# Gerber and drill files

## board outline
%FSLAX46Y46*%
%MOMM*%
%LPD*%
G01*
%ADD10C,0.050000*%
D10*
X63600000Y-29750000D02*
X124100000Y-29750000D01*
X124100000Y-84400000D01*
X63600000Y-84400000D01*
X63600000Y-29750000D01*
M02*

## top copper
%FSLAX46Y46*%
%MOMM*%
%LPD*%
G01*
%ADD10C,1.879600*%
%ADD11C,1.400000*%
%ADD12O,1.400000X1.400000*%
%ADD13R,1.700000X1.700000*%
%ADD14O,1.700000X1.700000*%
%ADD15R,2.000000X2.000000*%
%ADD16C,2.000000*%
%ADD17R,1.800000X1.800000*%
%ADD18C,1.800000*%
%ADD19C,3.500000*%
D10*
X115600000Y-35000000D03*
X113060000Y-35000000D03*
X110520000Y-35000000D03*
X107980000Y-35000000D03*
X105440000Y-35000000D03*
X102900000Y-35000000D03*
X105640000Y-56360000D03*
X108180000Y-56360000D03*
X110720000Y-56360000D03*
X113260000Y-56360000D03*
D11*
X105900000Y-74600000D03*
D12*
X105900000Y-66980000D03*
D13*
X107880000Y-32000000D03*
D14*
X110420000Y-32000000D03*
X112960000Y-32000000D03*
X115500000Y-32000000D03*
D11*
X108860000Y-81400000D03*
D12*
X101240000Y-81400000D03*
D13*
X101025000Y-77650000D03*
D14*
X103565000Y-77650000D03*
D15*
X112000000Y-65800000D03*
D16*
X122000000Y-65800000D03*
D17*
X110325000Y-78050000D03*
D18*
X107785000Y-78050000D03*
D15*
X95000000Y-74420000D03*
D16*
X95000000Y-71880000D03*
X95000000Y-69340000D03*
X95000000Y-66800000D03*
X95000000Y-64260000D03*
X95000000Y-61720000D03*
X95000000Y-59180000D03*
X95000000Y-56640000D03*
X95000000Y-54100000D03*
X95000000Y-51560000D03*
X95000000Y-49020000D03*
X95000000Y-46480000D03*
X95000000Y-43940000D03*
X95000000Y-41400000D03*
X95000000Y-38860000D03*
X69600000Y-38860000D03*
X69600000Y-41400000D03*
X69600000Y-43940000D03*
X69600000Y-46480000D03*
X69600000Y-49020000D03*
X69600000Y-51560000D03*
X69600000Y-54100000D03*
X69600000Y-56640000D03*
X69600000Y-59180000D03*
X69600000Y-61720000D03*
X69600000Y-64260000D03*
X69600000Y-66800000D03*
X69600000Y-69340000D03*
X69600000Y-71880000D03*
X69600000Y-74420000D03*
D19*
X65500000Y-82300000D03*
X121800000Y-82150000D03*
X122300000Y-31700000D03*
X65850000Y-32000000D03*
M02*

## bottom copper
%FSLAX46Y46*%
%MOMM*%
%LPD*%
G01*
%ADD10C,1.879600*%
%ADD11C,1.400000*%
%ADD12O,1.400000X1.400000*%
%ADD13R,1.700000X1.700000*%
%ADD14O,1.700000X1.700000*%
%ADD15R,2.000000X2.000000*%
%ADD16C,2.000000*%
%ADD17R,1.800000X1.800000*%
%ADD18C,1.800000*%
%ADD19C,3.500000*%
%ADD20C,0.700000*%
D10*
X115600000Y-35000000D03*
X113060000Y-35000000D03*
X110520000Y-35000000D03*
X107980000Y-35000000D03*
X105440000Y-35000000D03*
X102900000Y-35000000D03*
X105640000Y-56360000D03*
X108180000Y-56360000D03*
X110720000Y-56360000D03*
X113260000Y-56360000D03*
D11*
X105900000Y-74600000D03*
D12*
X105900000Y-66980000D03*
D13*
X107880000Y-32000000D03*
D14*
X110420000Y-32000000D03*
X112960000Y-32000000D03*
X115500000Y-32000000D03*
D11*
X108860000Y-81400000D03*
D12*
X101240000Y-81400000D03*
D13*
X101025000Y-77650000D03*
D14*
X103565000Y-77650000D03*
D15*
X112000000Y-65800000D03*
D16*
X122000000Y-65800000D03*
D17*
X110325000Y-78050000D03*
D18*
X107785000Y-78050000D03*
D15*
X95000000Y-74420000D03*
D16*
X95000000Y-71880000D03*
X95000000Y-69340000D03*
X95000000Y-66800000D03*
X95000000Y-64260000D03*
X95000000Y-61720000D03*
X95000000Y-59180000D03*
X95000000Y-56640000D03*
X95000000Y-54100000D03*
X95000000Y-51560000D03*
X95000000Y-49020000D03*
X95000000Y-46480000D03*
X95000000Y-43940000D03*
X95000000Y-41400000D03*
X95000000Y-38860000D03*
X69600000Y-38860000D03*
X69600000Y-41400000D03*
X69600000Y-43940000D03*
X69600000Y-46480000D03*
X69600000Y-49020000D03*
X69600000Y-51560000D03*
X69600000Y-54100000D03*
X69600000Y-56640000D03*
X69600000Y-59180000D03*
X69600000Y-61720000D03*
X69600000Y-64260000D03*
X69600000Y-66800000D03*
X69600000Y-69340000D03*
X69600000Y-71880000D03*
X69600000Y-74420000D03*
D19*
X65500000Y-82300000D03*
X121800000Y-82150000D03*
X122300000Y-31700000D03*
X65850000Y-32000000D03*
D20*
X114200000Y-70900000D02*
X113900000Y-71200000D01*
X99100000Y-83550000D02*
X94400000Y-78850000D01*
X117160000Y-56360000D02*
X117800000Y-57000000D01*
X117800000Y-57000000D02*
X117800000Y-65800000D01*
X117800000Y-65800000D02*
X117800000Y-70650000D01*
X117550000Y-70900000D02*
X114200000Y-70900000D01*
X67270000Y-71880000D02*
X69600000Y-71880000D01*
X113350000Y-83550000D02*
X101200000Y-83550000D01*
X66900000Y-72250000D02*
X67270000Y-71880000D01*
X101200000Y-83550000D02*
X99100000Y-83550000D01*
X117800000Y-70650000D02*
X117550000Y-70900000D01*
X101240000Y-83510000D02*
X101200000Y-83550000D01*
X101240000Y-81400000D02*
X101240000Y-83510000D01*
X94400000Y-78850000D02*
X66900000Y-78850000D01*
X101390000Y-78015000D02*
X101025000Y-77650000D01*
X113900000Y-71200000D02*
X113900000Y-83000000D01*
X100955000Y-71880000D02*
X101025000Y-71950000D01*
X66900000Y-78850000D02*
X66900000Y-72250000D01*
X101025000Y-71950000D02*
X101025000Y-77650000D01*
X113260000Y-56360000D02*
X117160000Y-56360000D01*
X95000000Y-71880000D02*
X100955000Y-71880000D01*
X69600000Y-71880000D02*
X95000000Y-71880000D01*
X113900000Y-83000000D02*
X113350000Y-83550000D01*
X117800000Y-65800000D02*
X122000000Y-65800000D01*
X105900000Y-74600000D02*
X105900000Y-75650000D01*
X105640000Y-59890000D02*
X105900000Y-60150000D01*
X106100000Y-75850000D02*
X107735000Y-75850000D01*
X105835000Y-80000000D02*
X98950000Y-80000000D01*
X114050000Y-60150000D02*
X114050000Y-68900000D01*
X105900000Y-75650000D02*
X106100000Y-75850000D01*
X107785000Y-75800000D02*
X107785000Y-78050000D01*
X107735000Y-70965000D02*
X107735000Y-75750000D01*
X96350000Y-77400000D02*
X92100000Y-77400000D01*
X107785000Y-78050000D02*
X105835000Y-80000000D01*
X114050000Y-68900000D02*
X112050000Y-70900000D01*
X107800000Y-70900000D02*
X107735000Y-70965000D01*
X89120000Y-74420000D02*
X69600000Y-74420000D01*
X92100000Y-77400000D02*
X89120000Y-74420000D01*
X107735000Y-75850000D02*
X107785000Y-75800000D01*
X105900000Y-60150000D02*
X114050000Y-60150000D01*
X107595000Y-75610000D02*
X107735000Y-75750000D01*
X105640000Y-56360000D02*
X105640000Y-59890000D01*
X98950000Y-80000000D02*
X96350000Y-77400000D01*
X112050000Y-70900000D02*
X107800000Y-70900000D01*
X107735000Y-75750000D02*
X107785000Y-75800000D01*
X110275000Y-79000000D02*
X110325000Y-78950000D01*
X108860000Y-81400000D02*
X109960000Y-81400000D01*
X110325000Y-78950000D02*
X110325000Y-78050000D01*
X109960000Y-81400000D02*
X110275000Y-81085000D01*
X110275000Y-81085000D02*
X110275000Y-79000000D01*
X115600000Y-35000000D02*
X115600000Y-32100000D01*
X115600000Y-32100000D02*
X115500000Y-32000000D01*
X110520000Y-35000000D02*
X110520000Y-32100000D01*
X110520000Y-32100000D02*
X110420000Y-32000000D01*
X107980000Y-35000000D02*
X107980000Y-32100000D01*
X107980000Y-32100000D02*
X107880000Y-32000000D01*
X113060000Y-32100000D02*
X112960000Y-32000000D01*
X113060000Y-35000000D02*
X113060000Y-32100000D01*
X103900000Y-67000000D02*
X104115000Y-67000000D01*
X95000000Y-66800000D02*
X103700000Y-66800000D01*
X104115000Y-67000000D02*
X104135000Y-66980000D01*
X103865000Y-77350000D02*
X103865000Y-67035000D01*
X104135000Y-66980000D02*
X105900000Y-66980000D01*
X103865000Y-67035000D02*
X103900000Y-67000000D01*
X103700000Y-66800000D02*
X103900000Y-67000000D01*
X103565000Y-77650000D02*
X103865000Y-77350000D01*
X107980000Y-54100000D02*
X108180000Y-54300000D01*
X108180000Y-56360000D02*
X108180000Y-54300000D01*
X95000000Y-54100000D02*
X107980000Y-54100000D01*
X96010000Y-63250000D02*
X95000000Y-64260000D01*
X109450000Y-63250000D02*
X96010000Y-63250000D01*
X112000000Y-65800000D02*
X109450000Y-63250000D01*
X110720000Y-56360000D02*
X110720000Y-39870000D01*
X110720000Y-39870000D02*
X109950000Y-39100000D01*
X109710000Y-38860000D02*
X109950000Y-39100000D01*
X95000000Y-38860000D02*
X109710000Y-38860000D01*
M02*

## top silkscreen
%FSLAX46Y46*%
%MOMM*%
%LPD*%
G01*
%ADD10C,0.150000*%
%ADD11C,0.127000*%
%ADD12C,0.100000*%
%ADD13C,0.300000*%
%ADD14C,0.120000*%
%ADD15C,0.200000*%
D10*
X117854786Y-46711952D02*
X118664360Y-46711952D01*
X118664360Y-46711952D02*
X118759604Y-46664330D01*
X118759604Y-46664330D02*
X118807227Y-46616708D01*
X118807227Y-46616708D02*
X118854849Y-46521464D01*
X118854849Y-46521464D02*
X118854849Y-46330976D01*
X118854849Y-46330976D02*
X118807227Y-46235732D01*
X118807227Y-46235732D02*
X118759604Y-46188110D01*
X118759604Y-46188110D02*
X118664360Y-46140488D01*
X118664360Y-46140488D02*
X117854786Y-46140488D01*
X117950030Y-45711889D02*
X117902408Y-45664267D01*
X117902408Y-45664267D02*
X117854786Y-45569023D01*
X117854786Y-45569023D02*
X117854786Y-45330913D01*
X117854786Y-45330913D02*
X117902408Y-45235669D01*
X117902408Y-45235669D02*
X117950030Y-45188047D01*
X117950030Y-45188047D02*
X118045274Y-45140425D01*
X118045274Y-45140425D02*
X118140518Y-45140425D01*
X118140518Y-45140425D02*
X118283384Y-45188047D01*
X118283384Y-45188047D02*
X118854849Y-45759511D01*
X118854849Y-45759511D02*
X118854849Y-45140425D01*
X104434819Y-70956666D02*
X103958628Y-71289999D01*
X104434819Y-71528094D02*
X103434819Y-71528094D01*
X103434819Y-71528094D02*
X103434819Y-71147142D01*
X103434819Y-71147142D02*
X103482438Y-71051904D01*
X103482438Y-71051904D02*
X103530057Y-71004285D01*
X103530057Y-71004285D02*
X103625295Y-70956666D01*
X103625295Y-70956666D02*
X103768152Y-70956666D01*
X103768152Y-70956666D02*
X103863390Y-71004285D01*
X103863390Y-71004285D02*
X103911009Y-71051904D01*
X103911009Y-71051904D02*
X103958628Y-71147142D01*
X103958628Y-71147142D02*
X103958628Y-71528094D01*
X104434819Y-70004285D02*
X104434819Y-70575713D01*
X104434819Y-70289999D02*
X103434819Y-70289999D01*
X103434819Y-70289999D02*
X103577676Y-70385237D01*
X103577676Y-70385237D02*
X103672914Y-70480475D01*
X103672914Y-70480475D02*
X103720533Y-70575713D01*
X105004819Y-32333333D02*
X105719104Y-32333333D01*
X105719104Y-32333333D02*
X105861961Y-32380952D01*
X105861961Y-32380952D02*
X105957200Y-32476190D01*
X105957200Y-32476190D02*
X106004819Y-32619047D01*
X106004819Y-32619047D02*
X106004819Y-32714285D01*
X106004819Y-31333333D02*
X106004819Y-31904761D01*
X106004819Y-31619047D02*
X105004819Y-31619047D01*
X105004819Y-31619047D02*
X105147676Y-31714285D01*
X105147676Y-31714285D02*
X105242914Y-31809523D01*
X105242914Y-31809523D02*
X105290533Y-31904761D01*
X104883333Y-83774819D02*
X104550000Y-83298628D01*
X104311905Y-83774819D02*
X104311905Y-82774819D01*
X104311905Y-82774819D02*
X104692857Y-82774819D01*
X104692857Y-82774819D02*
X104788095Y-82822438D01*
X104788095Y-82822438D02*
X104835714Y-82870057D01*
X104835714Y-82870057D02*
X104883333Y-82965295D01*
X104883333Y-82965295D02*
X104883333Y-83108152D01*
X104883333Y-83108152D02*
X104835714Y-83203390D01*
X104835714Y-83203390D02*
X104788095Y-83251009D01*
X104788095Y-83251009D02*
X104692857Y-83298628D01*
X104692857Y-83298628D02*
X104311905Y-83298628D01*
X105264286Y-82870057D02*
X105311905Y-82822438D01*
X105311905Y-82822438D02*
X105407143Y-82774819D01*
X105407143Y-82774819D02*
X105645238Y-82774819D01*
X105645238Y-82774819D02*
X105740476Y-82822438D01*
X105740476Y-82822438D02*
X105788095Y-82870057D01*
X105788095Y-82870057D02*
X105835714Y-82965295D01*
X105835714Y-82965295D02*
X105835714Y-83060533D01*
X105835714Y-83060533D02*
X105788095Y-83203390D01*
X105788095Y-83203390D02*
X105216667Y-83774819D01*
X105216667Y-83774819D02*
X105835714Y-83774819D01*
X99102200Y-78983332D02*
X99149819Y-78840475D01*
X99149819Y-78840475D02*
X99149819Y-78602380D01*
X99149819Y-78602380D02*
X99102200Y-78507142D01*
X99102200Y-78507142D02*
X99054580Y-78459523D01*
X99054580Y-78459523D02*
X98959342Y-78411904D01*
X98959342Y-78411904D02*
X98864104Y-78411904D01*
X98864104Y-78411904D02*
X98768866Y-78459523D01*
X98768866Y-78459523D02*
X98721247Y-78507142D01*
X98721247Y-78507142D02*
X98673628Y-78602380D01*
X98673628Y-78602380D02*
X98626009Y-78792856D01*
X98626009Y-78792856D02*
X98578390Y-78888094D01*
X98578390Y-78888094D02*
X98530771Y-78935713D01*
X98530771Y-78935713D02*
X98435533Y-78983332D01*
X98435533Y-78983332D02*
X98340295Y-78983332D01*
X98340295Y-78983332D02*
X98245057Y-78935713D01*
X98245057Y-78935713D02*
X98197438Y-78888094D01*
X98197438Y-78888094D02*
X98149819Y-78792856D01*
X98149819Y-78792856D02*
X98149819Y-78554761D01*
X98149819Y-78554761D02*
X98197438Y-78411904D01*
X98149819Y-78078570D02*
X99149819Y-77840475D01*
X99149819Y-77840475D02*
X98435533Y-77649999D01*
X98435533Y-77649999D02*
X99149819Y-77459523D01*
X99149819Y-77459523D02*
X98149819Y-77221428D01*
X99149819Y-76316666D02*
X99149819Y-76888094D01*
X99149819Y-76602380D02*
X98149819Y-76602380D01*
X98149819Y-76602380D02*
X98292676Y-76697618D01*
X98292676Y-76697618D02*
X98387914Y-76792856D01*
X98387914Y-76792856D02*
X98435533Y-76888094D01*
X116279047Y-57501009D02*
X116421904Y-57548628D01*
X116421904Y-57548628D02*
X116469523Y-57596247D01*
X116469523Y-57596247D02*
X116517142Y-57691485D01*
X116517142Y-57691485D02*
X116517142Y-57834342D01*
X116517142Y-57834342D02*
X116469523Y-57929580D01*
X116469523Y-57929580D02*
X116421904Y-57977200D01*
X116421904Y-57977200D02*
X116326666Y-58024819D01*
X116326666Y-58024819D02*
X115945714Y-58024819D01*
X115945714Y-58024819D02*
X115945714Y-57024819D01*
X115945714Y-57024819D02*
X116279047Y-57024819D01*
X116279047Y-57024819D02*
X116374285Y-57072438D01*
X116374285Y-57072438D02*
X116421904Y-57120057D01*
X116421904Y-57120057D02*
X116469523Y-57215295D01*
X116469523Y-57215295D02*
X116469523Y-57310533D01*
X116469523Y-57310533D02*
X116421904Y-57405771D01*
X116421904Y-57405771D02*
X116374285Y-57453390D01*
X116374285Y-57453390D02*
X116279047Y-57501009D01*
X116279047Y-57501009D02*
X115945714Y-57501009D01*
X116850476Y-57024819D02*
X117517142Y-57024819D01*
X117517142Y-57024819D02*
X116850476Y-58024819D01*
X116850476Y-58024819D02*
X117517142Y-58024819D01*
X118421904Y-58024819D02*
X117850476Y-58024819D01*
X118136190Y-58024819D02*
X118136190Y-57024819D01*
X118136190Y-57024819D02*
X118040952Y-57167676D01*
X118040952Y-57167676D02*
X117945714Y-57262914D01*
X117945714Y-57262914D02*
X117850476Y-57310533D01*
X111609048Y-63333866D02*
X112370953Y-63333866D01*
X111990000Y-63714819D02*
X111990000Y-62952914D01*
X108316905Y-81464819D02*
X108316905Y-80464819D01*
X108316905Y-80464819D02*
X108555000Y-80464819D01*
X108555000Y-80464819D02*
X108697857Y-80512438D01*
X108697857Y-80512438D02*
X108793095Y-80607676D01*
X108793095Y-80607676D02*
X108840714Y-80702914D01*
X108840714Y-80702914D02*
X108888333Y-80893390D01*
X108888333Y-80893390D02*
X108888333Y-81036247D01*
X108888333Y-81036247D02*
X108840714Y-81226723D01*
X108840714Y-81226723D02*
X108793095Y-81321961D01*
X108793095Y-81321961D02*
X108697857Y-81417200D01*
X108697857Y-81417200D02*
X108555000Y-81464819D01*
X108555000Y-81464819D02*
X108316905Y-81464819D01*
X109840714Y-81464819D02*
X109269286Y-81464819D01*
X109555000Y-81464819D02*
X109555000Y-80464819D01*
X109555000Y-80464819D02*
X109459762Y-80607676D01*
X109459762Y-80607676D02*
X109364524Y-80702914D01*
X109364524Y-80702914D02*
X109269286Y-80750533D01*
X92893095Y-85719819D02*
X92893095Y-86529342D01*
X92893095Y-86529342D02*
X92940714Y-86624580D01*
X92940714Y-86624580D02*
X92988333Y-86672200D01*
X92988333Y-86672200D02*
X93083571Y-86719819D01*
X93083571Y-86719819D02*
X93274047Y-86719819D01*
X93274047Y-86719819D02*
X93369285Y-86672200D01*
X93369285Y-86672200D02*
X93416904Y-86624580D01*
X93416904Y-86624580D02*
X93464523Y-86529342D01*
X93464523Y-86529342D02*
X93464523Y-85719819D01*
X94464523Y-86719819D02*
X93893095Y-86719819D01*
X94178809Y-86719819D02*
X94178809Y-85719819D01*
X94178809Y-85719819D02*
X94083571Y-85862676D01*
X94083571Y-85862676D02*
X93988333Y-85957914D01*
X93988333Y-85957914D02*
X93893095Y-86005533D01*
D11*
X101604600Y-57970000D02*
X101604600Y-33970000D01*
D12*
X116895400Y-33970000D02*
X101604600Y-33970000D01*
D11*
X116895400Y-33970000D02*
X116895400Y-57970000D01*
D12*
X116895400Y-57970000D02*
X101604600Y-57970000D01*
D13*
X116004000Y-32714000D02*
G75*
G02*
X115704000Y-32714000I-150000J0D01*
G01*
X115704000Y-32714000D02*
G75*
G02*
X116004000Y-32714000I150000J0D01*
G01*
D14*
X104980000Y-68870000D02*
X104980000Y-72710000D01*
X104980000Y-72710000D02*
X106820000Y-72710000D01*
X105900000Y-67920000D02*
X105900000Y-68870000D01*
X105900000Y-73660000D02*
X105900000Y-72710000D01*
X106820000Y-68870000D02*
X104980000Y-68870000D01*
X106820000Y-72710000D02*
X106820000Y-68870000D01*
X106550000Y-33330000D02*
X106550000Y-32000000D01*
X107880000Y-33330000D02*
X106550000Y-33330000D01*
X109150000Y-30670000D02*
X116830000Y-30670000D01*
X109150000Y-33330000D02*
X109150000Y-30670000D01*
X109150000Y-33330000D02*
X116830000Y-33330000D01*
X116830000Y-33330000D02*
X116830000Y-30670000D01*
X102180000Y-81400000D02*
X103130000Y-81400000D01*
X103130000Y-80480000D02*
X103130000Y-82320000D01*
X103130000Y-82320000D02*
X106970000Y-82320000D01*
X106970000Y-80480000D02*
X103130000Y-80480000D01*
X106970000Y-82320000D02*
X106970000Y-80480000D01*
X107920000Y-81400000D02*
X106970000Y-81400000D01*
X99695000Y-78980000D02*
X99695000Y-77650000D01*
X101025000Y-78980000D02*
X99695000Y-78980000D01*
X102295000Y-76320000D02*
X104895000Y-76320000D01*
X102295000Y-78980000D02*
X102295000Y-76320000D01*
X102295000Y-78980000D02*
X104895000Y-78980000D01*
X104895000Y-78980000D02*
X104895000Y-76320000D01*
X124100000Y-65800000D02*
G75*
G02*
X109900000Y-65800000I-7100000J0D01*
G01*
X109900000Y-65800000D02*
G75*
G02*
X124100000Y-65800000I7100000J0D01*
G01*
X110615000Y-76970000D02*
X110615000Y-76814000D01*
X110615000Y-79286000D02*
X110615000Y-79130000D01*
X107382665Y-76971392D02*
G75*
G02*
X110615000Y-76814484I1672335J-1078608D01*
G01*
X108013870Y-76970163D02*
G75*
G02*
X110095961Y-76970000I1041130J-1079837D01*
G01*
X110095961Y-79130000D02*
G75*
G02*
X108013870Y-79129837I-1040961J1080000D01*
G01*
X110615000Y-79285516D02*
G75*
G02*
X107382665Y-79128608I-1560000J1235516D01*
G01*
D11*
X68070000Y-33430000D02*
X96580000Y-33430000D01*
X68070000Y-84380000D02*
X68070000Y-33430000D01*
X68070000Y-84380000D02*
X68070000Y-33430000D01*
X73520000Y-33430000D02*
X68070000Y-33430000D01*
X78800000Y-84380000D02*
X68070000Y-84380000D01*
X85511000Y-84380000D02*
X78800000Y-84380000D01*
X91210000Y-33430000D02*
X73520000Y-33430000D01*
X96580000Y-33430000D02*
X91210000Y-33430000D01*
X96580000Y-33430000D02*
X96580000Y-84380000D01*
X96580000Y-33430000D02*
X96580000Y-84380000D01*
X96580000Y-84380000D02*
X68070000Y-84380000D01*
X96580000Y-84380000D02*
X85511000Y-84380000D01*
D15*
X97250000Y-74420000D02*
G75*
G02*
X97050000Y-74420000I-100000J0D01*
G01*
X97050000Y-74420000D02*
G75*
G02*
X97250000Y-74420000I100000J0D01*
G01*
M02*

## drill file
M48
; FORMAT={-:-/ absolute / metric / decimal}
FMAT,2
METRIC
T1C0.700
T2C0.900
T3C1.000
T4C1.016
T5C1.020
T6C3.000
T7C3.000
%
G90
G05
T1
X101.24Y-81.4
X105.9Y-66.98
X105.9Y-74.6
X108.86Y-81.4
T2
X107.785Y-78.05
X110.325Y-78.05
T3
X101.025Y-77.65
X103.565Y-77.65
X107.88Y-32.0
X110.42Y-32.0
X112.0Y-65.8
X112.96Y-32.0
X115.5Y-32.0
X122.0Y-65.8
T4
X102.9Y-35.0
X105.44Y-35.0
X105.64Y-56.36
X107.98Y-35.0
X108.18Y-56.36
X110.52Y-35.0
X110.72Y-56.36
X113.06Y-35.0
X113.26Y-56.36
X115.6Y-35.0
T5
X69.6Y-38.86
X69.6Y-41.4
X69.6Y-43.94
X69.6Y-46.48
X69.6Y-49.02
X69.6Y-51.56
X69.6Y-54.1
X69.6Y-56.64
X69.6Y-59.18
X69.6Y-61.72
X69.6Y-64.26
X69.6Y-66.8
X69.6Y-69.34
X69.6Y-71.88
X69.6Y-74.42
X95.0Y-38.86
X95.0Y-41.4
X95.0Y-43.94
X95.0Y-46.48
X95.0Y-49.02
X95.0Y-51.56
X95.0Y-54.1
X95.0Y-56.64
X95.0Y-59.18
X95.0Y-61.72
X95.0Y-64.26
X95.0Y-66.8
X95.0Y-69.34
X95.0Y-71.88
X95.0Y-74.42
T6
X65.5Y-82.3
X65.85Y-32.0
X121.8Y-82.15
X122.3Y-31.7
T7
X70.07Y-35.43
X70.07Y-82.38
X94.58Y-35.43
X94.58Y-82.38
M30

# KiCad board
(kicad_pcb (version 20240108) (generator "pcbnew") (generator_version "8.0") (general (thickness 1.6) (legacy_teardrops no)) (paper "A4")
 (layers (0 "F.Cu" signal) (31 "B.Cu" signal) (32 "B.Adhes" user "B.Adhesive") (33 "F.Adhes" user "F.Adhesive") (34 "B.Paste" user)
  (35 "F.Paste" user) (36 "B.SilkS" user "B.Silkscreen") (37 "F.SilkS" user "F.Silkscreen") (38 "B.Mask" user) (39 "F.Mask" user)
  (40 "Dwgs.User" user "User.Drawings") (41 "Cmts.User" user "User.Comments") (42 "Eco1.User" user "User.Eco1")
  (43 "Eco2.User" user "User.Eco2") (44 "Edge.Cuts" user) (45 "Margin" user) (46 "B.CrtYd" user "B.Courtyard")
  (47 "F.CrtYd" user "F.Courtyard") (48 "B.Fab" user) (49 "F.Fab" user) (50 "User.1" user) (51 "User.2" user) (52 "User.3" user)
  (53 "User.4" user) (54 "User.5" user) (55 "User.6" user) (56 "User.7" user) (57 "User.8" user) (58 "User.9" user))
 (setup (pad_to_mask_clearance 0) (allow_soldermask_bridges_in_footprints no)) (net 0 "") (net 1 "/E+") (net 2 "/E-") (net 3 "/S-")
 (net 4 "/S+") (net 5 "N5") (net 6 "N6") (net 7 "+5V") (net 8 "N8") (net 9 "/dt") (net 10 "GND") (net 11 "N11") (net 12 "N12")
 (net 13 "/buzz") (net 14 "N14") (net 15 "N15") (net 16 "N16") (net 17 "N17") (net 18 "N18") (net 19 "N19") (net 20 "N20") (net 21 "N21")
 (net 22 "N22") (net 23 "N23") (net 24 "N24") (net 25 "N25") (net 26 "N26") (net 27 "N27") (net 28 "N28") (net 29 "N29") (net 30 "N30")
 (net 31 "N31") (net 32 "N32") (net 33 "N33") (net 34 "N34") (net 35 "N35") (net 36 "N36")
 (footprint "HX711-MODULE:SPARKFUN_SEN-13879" (layer "F.Cu") (at 110.52 48.97 -90)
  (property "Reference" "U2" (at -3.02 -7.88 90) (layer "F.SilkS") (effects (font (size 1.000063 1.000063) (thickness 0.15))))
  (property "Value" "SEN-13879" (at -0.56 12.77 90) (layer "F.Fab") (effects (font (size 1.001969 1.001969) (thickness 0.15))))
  (fp_line (start 9 8.9154) (end -15 8.9154) (stroke (width 0.127) (type solid)) (layer "F.SilkS"))
  (fp_line (start -15 -6.3754) (end -15 8.9154) (stroke (width 0.1) (type default)) (layer "F.SilkS"))
  (fp_line (start -15 -6.3754) (end 9 -6.3754) (stroke (width 0.127) (type solid)) (layer "F.SilkS"))
  (fp_line (start 9 -6.3754) (end 9 8.9154) (stroke (width 0.1) (type default)) (layer "F.SilkS"))
  (fp_circle (center -16.256 -5.334) (end -16.106 -5.334) (stroke (width 0.3) (type solid)) (fill none) (layer "F.SilkS"))
  (pad "1" thru_hole circle (at -13.97 -5.08 270) (size 1.8796 1.8796) (drill 1.016) (layers "*.Cu" "*.Mask") (remove_unused_layers no)
   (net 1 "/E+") (solder_mask_margin 0.102))
  (pad "2" thru_hole circle (at -13.97 -2.54 270) (size 1.8796 1.8796) (drill 1.016) (layers "*.Cu" "*.Mask") (remove_unused_layers no)
   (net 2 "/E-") (solder_mask_margin 0.102))
  (pad "3" thru_hole circle (at -13.97 0 270) (size 1.8796 1.8796) (drill 1.016) (layers "*.Cu" "*.Mask") (remove_unused_layers no)
   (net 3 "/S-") (solder_mask_margin 0.102))
  (pad "4" thru_hole circle (at -13.97 2.54 270) (size 1.8796 1.8796) (drill 1.016) (layers "*.Cu" "*.Mask") (remove_unused_layers no)
   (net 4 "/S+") (solder_mask_margin 0.102))
  (pad "5" thru_hole circle (at -13.97 5.08 270) (size 1.8796 1.8796) (drill 1.016) (layers "*.Cu" "*.Mask") (remove_unused_layers no)
   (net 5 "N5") (solder_mask_margin 0.102))
  (pad "6" thru_hole circle (at -13.97 7.62 270) (size 1.8796 1.8796) (drill 1.016) (layers "*.Cu" "*.Mask") (remove_unused_layers no)
   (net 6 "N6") (solder_mask_margin 0.102))
  (pad "7" thru_hole circle (at 7.39 4.88 270) (size 1.8796 1.8796) (drill 1.016) (layers "*.Cu" "*.Mask") (remove_unused_layers no)
   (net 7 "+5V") (solder_mask_margin 0.102))
  (pad "8" thru_hole circle (at 7.39 2.34 270) (size 1.8796 1.8796) (drill 1.016) (layers "*.Cu" "*.Mask") (remove_unused_layers no)
   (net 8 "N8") (solder_mask_margin 0.102))
  (pad "9" thru_hole circle (at 7.39 -0.2 270) (size 1.8796 1.8796) (drill 1.016) (layers "*.Cu" "*.Mask") (remove_unused_layers no)
   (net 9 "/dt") (solder_mask_margin 0.102))
  (pad "10" thru_hole circle (at 7.39 -2.74 270) (size 1.8796 1.8796) (drill 1.016) (layers "*.Cu" "*.Mask") (remove_unused_layers no)
   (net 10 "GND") (solder_mask_margin 0.102)))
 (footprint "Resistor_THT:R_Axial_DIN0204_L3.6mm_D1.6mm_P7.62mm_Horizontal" (layer "F.Cu") (at 105.9 74.6 90)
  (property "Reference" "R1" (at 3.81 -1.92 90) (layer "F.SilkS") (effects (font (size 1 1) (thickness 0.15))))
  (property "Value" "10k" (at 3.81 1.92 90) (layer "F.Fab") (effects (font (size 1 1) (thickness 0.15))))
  (fp_line (start 5.73 -0.92) (end 1.89 -0.92) (stroke (width 0.12) (type solid)) (layer "F.SilkS"))
  (fp_line (start 1.89 -0.92) (end 1.89 0.92) (stroke (width 0.12) (type solid)) (layer "F.SilkS"))
  (fp_line (start 6.68 0) (end 5.73 0) (stroke (width 0.12) (type solid)) (layer "F.SilkS"))
  (fp_line (start 0.94 0) (end 1.89 0) (stroke (width 0.12) (type solid)) (layer "F.SilkS"))
  (fp_line (start 5.73 0.92) (end 5.73 -0.92) (stroke (width 0.12) (type solid)) (layer "F.SilkS"))
  (fp_line (start 1.89 0.92) (end 5.73 0.92) (stroke (width 0.12) (type solid)) (layer "F.SilkS"))
  (pad "1" thru_hole circle (at 0 0 90) (size 1.4 1.4) (drill 0.7) (layers "*.Cu" "*.Mask") (remove_unused_layers no) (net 7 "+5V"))
  (pad "2" thru_hole oval (at 7.62 0 90) (size 1.4 1.4) (drill 0.7) (layers "*.Cu" "*.Mask") (remove_unused_layers no) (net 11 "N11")))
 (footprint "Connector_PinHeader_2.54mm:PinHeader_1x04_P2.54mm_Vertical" (layer "F.Cu") (at 107.88 32 90)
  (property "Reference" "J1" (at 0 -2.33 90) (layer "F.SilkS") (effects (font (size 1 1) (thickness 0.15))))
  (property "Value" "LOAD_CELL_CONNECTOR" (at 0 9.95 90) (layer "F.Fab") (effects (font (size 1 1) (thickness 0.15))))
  (fp_line (start -1.33 -1.33) (end 0 -1.33) (stroke (width 0.12) (type solid)) (layer "F.SilkS"))
  (fp_line (start -1.33 0) (end -1.33 -1.33) (stroke (width 0.12) (type solid)) (layer "F.SilkS"))
  (fp_line (start 1.33 1.27) (end 1.33 8.95) (stroke (width 0.12) (type solid)) (layer "F.SilkS"))
  (fp_line (start -1.33 1.27) (end 1.33 1.27) (stroke (width 0.12) (type solid)) (layer "F.SilkS"))
  (fp_line (start -1.33 1.27) (end -1.33 8.95) (stroke (width 0.12) (type solid)) (layer "F.SilkS"))
  (fp_line (start -1.33 8.95) (end 1.33 8.95) (stroke (width 0.12) (type solid)) (layer "F.SilkS"))
  (pad "1" thru_hole rect (at 0 0 90) (size 1.7 1.7) (drill 1) (layers "*.Cu" "*.Mask") (remove_unused_layers no) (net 4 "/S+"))
  (pad "2" thru_hole oval (at 0 2.54 90) (size 1.7 1.7) (drill 1) (layers "*.Cu" "*.Mask") (remove_unused_layers no) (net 3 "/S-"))
  (pad "3" thru_hole oval (at 0 5.08 90) (size 1.7 1.7) (drill 1) (layers "*.Cu" "*.Mask") (remove_unused_layers no) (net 2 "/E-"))
  (pad "4" thru_hole oval (at 0 7.62 90) (size 1.7 1.7) (drill 1) (layers "*.Cu" "*.Mask") (remove_unused_layers no) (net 1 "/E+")))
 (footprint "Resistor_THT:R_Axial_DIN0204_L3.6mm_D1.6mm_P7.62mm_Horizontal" (layer "F.Cu") (at 108.86 81.4 180)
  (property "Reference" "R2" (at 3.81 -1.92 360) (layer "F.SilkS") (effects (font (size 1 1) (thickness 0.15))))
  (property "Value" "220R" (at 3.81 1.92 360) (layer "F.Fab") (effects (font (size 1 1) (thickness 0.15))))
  (fp_line (start 6.68 0) (end 5.73 0) (stroke (width 0.12) (type solid)) (layer "F.SilkS"))
  (fp_line (start 5.73 0.92) (end 5.73 -0.92) (stroke (width 0.12) (type solid)) (layer "F.SilkS"))
  (fp_line (start 5.73 -0.92) (end 1.89 -0.92) (stroke (width 0.12) (type solid)) (layer "F.SilkS"))
  (fp_line (start 1.89 0.92) (end 5.73 0.92) (stroke (width 0.12) (type solid)) (layer "F.SilkS"))
  (fp_line (start 1.89 -0.92) (end 1.89 0.92) (stroke (width 0.12) (type solid)) (layer "F.SilkS"))
  (fp_line (start 0.94 0) (end 1.89 0) (stroke (width 0.12) (type solid)) (layer "F.SilkS"))
  (pad "1" thru_hole circle (at 0 0 180) (size 1.4 1.4) (drill 0.7) (layers "*.Cu" "*.Mask") (remove_unused_layers no) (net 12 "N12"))
  (pad "2" thru_hole oval (at 7.62 0 180) (size 1.4 1.4) (drill 0.7) (layers "*.Cu" "*.Mask") (remove_unused_layers no) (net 10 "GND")))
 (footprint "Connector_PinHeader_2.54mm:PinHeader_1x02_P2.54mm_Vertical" (layer "F.Cu") (at 101.025 77.65 90)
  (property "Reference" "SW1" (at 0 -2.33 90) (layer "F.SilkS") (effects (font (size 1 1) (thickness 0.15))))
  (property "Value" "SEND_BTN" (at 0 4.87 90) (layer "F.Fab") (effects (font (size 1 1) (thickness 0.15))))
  (fp_line (start -1.33 -1.33) (end 0 -1.33) (stroke (width 0.12) (type solid)) (layer "F.SilkS"))
  (fp_line (start -1.33 0) (end -1.33 -1.33) (stroke (width 0.12) (type solid)) (layer "F.SilkS"))
  (fp_line (start 1.33 1.27) (end 1.33 3.87) (stroke (width 0.12) (type solid)) (layer "F.SilkS"))
  (fp_line (start -1.33 1.27) (end 1.33 1.27) (stroke (width 0.12) (type solid)) (layer "F.SilkS"))
  (fp_line (start -1.33 1.27) (end -1.33 3.87) (stroke (width 0.12) (type solid)) (layer "F.SilkS"))
  (fp_line (start -1.33 3.87) (end 1.33 3.87) (stroke (width 0.12) (type solid)) (layer "F.SilkS"))
  (pad "1" thru_hole rect (at 0 0 90) (size 1.7 1.7) (drill 1) (layers "*.Cu" "*.Mask") (remove_unused_layers no) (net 10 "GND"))
  (pad "2" thru_hole oval (at 0 2.54 90) (size 1.7 1.7) (drill 1) (layers "*.Cu" "*.Mask") (remove_unused_layers no) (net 11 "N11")))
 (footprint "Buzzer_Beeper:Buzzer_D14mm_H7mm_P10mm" (layer "F.Cu") (at 112 65.8)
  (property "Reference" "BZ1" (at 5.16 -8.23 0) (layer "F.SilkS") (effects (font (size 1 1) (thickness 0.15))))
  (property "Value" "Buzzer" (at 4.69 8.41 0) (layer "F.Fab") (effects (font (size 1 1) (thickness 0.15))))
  (fp_circle (center 5 0) (end 12.1 0) (stroke (width 0.12) (type solid)) (fill none) (layer "F.SilkS"))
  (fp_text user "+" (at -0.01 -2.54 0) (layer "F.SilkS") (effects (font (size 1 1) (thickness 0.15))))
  (pad "1" thru_hole rect (at 0 0) (size 2 2) (drill 1) (layers "*.Cu" "*.Mask") (remove_unused_layers no) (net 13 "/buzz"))
  (pad "2" thru_hole circle (at 10 0) (size 2 2) (drill 1) (layers "*.Cu" "*.Mask") (remove_unused_layers no) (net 10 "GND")))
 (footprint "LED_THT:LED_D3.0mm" (layer "F.Cu") (at 110.325 78.05 180)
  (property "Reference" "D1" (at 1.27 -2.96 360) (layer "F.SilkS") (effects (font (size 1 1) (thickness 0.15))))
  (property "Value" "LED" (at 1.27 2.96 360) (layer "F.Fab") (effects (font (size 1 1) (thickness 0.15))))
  (fp_line (start -0.29 1.08) (end -0.29 1.236) (stroke (width 0.12) (type solid)) (layer "F.SilkS"))
  (fp_line (start -0.29 -1.236) (end -0.29 -1.08) (stroke (width 0.12) (type solid)) (layer "F.SilkS"))
  (fp_arc (start 2.942335 1.078608) (mid 1.366487 1.987659) (end -0.29 1.235516) (stroke (width 0.12) (type solid)) (layer "F.SilkS"))
  (fp_arc (start 2.31113 1.079837) (mid 1.270117 1.5) (end 0.229039 1.08) (stroke (width 0.12) (type solid)) (layer "F.SilkS"))
  (fp_arc (start 0.229039 -1.08) (mid 1.270117 -1.5) (end 2.31113 -1.079837) (stroke (width 0.12) (type solid)) (layer "F.SilkS"))
  (fp_arc (start -0.29 -1.235516) (mid 1.366487 -1.987659) (end 2.942335 -1.078608) (stroke (width 0.12) (type solid)) (layer "F.SilkS"))
  (pad "1" thru_hole rect (at 0 0 180) (size 1.8 1.8) (drill 0.9) (layers "*.Cu" "*.Mask") (remove_unused_layers no) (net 12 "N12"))
  (pad "2" thru_hole circle (at 2.54 0 180) (size 1.8 1.8) (drill 0.9) (layers "*.Cu" "*.Mask") (remove_unused_layers no) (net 7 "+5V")))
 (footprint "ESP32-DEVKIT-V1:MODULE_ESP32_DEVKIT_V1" (layer "F.Cu") (at 82.3 58.905 180)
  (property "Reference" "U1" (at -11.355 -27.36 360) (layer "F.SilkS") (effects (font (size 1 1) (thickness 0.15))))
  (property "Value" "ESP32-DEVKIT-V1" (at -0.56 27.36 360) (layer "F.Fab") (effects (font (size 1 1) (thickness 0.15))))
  (fp_line (start 14.23 25.475) (end -14.28 25.475) (stroke (width 0.127) (type solid)) (layer "F.SilkS"))
  (fp_line (start 14.23 -25.475) (end 14.23 25.475) (stroke (width 0.127) (type solid)) (layer "F.SilkS"))
  (fp_line (start 14.23 -25.475) (end 14.23 25.475) (stroke (width 0.127) (type solid)) (layer "F.SilkS"))
  (fp_line (start 8.78 25.475) (end 14.23 25.475) (stroke (width 0.127) (type solid)) (layer "F.SilkS"))
  (fp_line (start 3.5 -25.475) (end 14.23 -25.475) (stroke (width 0.127) (type solid)) (layer "F.SilkS"))
  (fp_line (start -3.211 -25.475) (end 3.5 -25.475) (stroke (width 0.127) (type solid)) (layer "F.SilkS"))
  (fp_line (start -8.91 25.475) (end 8.78 25.475) (stroke (width 0.127) (type solid)) (layer "F.SilkS"))
  (fp_line (start -14.28 25.475) (end -8.91 25.475) (stroke (width 0.127) (type solid)) (layer "F.SilkS"))
  (fp_line (start -14.28 25.475) (end -14.28 -25.475) (stroke (width 0.127) (type solid)) (layer "F.SilkS"))
  (fp_line (start -14.28 25.475) (end -14.28 -25.475) (stroke (width 0.127) (type solid)) (layer "F.SilkS"))
  (fp_line (start -14.28 -25.475) (end 14.23 -25.475) (stroke (width 0.127) (type solid)) (layer "F.SilkS"))
  (fp_line (start -14.28 -25.475) (end -3.211 -25.475) (stroke (width 0.127) (type solid)) (layer "F.SilkS"))
  (fp_circle (center -14.85 -15.515) (end -14.75 -15.515) (stroke (width 0.2) (type solid)) (fill none) (layer "F.SilkS"))
  (pad "" np_thru_hole circle (at -12.28 -23.475 180) (size 3 3) (drill 3) (layers "*.Cu" "*.Mask"))
  (pad "" np_thru_hole circle (at -12.28 23.475 180) (size 3 3) (drill 3) (layers "*.Cu" "*.Mask"))
  (pad "" np_thru_hole circle (at 12.23 -23.475 180) (size 3 3) (drill 3) (layers "*.Cu" "*.Mask"))
  (pad "" np_thru_hole circle (at 12.23 23.475 180) (size 3 3) (drill 3) (layers "*.Cu" "*.Mask"))
  (pad "1" thru_hole rect (at -12.7 -15.515 180) (size 2 2) (drill 1.02) (layers "*.Cu" "*.Mask") (remove_unused_layers no) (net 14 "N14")
   (solder_mask_margin 0.102))
  (pad "2" thru_hole circle (at -12.7 -12.975 180) (size 2 2) (drill 1.02) (layers "*.Cu" "*.Mask") (remove_unused_layers no) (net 10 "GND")
   (solder_mask_margin 0.102))
  (pad "3" thru_hole circle (at -12.7 -10.435 180) (size 2 2) (drill 1.02) (layers "*.Cu" "*.Mask") (remove_unused_layers no) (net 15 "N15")
   (solder_mask_margin 0.102))
  (pad "4" thru_hole circle (at -12.7 -7.895 180) (size 2 2) (drill 1.02) (layers "*.Cu" "*.Mask") (remove_unused_layers no) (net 11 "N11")
   (solder_mask_margin 0.102))
  (pad "5" thru_hole circle (at -12.7 -5.355 180) (size 2 2) (drill 1.02) (layers "*.Cu" "*.Mask") (remove_unused_layers no)
   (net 13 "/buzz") (solder_mask_margin 0.102))
  (pad "6" thru_hole circle (at -12.7 -2.815 180) (size 2 2) (drill 1.02) (layers "*.Cu" "*.Mask") (remove_unused_layers no) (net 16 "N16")
   (solder_mask_margin 0.102))
  (pad "7" thru_hole circle (at -12.7 -0.275 180) (size 2 2) (drill 1.02) (layers "*.Cu" "*.Mask") (remove_unused_layers no) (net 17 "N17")
   (solder_mask_margin 0.102))
  (pad "8" thru_hole circle (at -12.7 2.265 180) (size 2 2) (drill 1.02) (layers "*.Cu" "*.Mask") (remove_unused_layers no) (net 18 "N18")
   (solder_mask_margin 0.102))
  (pad "9" thru_hole circle (at -12.7 4.805 180) (size 2 2) (drill 1.02) (layers "*.Cu" "*.Mask") (remove_unused_layers no) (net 8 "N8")
   (solder_mask_margin 0.102))
  (pad "10" thru_hole circle (at -12.7 7.345 180) (size 2 2) (drill 1.02) (layers "*.Cu" "*.Mask") (remove_unused_layers no) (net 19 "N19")
   (solder_mask_margin 0.102))
  (pad "11" thru_hole circle (at -12.7 9.885 180) (size 2 2) (drill 1.02) (layers "*.Cu" "*.Mask") (remove_unused_layers no) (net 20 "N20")
   (solder_mask_margin 0.102))
  (pad "12" thru_hole circle (at -12.7 12.425 180) (size 2 2) (drill 1.02) (layers "*.Cu" "*.Mask") (remove_unused_layers no) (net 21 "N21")
   (solder_mask_margin 0.102))
  (pad "13" thru_hole circle (at -12.7 14.965 180) (size 2 2) (drill 1.02) (layers "*.Cu" "*.Mask") (remove_unused_layers no) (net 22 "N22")
   (solder_mask_margin 0.102))
  (pad "14" thru_hole circle (at -12.7 17.505 180) (size 2 2) (drill 1.02) (layers "*.Cu" "*.Mask") (remove_unused_layers no) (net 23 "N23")
   (solder_mask_margin 0.102))
  (pad "15" thru_hole circle (at -12.7 20.045 180) (size 2 2) (drill 1.02) (layers "*.Cu" "*.Mask") (remove_unused_layers no) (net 9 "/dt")
   (solder_mask_margin 0.102))
  (pad "16" thru_hole circle (at 12.7 20.045 180) (size 2 2) (drill 1.02) (layers "*.Cu" "*.Mask") (remove_unused_layers no) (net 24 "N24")
   (solder_mask_margin 0.102))
  (pad "17" thru_hole circle (at 12.7 17.505 180) (size 2 2) (drill 1.02) (layers "*.Cu" "*.Mask") (remove_unused_layers no) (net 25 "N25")
   (solder_mask_margin 0.102))
  (pad "18" thru_hole circle (at 12.7 14.965 180) (size 2 2) (drill 1.02) (layers "*.Cu" "*.Mask") (remove_unused_layers no) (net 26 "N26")
   (solder_mask_margin 0.102))
  (pad "19" thru_hole circle (at 12.7 12.425 180) (size 2 2) (drill 1.02) (layers "*.Cu" "*.Mask") (remove_unused_layers no) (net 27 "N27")
   (solder_mask_margin 0.102))
  (pad "20" thru_hole circle (at 12.7 9.885 180) (size 2 2) (drill 1.02) (layers "*.Cu" "*.Mask") (remove_unused_layers no) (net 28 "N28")
   (solder_mask_margin 0.102))
  (pad "21" thru_hole circle (at 12.7 7.345 180) (size 2 2) (drill 1.02) (layers "*.Cu" "*.Mask") (remove_unused_layers no) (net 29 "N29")
   (solder_mask_margin 0.102))
  (pad "22" thru_hole circle (at 12.7 4.805 180) (size 2 2) (drill 1.02) (layers "*.Cu" "*.Mask") (remove_unused_layers no) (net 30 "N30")
   (solder_mask_margin 0.102))
  (pad "23" thru_hole circle (at 12.7 2.265 180) (size 2 2) (drill 1.02) (layers "*.Cu" "*.Mask") (remove_unused_layers no) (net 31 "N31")
   (solder_mask_margin 0.102))
  (pad "24" thru_hole circle (at 12.7 -0.275 180) (size 2 2) (drill 1.02) (layers "*.Cu" "*.Mask") (remove_unused_layers no) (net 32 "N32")
   (solder_mask_margin 0.102))
  (pad "25" thru_hole circle (at 12.7 -2.815 180) (size 2 2) (drill 1.02) (layers "*.Cu" "*.Mask") (remove_unused_layers no) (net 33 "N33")
   (solder_mask_margin 0.102))
  (pad "26" thru_hole circle (at 12.7 -5.355 180) (size 2 2) (drill 1.02) (layers "*.Cu" "*.Mask") (remove_unused_layers no) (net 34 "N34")
   (solder_mask_margin 0.102))
  (pad "27" thru_hole circle (at 12.7 -7.895 180) (size 2 2) (drill 1.02) (layers "*.Cu" "*.Mask") (remove_unused_layers no) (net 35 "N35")
   (solder_mask_margin 0.102))
  (pad "28" thru_hole circle (at 12.7 -10.435 180) (size 2 2) (drill 1.02) (layers "*.Cu" "*.Mask") (remove_unused_layers no) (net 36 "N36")
   (solder_mask_margin 0.102))
  (pad "29" thru_hole circle (at 12.7 -12.975 180) (size 2 2) (drill 1.02) (layers "*.Cu" "*.Mask") (remove_unused_layers no) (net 10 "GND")
   (solder_mask_margin 0.102))
  (pad "30" thru_hole circle (at 12.7 -15.515 180) (size 2 2) (drill 1.02) (layers "*.Cu" "*.Mask") (remove_unused_layers no) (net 7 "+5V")
   (solder_mask_margin 0.102))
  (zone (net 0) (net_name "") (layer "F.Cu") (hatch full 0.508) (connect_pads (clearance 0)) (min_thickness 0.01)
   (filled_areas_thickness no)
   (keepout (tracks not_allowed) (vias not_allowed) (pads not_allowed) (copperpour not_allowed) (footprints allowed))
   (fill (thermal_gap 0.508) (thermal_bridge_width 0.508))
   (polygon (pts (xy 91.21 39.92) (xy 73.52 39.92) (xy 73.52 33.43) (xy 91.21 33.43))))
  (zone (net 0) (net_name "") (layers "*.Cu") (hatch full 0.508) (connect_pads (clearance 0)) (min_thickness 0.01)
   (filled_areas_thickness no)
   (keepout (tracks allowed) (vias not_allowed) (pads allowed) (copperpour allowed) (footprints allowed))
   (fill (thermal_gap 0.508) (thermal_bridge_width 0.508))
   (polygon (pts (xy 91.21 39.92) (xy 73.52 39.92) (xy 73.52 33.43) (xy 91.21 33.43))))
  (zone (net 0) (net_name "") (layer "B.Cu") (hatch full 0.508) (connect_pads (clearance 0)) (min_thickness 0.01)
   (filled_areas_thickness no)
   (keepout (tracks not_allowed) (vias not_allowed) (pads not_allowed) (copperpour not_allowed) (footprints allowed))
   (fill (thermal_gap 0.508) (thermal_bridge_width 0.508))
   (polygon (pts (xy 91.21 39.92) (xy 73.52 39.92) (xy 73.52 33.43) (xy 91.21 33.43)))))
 (gr_rect (start 63.6 29.75) (end 124.1 84.4) (stroke (width 0.05) (type default)) (fill none) (layer "Edge.Cuts"))
 (via (at 65.5 82.3) (size 3.5) (drill 3) (layers "F.Cu" "B.Cu") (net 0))
 (via (at 121.8 82.15) (size 3.5) (drill 3) (layers "F.Cu" "B.Cu") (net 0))
 (via (at 122.3 31.7) (size 3.5) (drill 3) (layers "F.Cu" "B.Cu") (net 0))
 (via (at 65.85 32) (size 3.5) (drill 3) (layers "F.Cu" "B.Cu") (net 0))
 (segment (start 114.2 70.9) (end 113.9 71.2) (width 0.7) (layer "B.Cu") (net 10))
 (segment (start 99.1 83.55) (end 94.4 78.85) (width 0.7) (layer "B.Cu") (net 10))
 (segment (start 117.16 56.36) (end 117.8 57) (width 0.7) (layer "B.Cu") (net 10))
 (segment (start 117.8 57) (end 117.8 65.8) (width 0.7) (layer "B.Cu") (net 10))
 (segment (start 117.8 65.8) (end 117.8 70.65) (width 0.7) (layer "B.Cu") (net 10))
 (segment (start 117.55 70.9) (end 114.2 70.9) (width 0.7) (layer "B.Cu") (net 10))
 (segment (start 67.27 71.88) (end 69.6 71.88) (width 0.7) (layer "B.Cu") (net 10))
 (segment (start 113.35 83.55) (end 101.2 83.55) (width 0.7) (layer "B.Cu") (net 10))
 (segment (start 66.9 72.25) (end 67.27 71.88) (width 0.7) (layer "B.Cu") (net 10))
 (segment (start 101.2 83.55) (end 99.1 83.55) (width 0.7) (layer "B.Cu") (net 10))
 (segment (start 117.8 70.65) (end 117.55 70.9) (width 0.7) (layer "B.Cu") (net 10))
 (segment (start 101.24 83.51) (end 101.2 83.55) (width 0.7) (layer "B.Cu") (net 10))
 (segment (start 101.24 81.4) (end 101.24 83.51) (width 0.7) (layer "B.Cu") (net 10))
 (segment (start 94.4 78.85) (end 66.9 78.85) (width 0.7) (layer "B.Cu") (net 10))
 (segment (start 101.39 78.015) (end 101.025 77.65) (width 0.7) (layer "B.Cu") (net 10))
 (segment (start 113.9 71.2) (end 113.9 83) (width 0.7) (layer "B.Cu") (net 10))
 (segment (start 100.955 71.88) (end 101.025 71.95) (width 0.7) (layer "B.Cu") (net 10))
 (segment (start 66.9 78.85) (end 66.9 72.25) (width 0.7) (layer "B.Cu") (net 10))
 (segment (start 101.025 71.95) (end 101.025 77.65) (width 0.7) (layer "B.Cu") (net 10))
 (segment (start 113.26 56.36) (end 117.16 56.36) (width 0.7) (layer "B.Cu") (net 10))
 (segment (start 95 71.88) (end 100.955 71.88) (width 0.7) (layer "B.Cu") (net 10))
 (segment (start 69.6 71.88) (end 95 71.88) (width 0.7) (layer "B.Cu") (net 10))
 (segment (start 113.9 83) (end 113.35 83.55) (width 0.7) (layer "B.Cu") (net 10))
 (segment (start 117.8 65.8) (end 122 65.8) (width 0.7) (layer "B.Cu") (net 10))
 (segment (start 105.9 74.6) (end 105.9 75.65) (width 0.7) (layer "B.Cu") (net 7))
 (segment (start 105.64 59.89) (end 105.9 60.15) (width 0.7) (layer "B.Cu") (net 7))
 (segment (start 106.1 75.85) (end 107.735 75.85) (width 0.7) (layer "B.Cu") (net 7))
 (segment (start 105.835 80) (end 98.95 80) (width 0.7) (layer "B.Cu") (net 7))
 (segment (start 114.05 60.15) (end 114.05 68.9) (width 0.7) (layer "B.Cu") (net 7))
 (segment (start 105.9 75.65) (end 106.1 75.85) (width 0.7) (layer "B.Cu") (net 7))
 (segment (start 107.785 75.8) (end 107.785 78.05) (width 0.7) (layer "B.Cu") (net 7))
 (segment (start 107.735 70.965) (end 107.735 75.75) (width 0.7) (layer "B.Cu") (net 7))
 (segment (start 96.35 77.4) (end 92.1 77.4) (width 0.7) (layer "B.Cu") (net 7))
 (segment (start 107.785 78.05) (end 105.835 80) (width 0.7) (layer "B.Cu") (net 7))
 (segment (start 114.05 68.9) (end 112.05 70.9) (width 0.7) (layer "B.Cu") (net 7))
 (segment (start 107.8 70.9) (end 107.735 70.965) (width 0.7) (layer "B.Cu") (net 7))
 (segment (start 89.12 74.42) (end 69.6 74.42) (width 0.7) (layer "B.Cu") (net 7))
 (segment (start 92.1 77.4) (end 89.12 74.42) (width 0.7) (layer "B.Cu") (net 7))
 (segment (start 107.735 75.85) (end 107.785 75.8) (width 0.7) (layer "B.Cu") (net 7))
 (segment (start 105.9 60.15) (end 114.05 60.15) (width 0.7) (layer "B.Cu") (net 7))
 (segment (start 107.595 75.61) (end 107.735 75.75) (width 0.7) (layer "B.Cu") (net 7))
 (segment (start 105.64 56.36) (end 105.64 59.89) (width 0.7) (layer "B.Cu") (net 7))
 (segment (start 98.95 80) (end 96.35 77.4) (width 0.7) (layer "B.Cu") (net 7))
 (segment (start 112.05 70.9) (end 107.8 70.9) (width 0.7) (layer "B.Cu") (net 7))
 (segment (start 107.735 75.75) (end 107.785 75.8) (width 0.7) (layer "B.Cu") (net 7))
 (segment (start 110.275 79) (end 110.325 78.95) (width 0.7) (layer "B.Cu") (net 12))
 (segment (start 108.86 81.4) (end 109.96 81.4) (width 0.7) (layer "B.Cu") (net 12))
 (segment (start 110.325 78.95) (end 110.325 78.05) (width 0.7) (layer "B.Cu") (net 12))
 (segment (start 109.96 81.4) (end 110.275 81.085) (width 0.7) (layer "B.Cu") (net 12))
 (segment (start 110.275 81.085) (end 110.275 79) (width 0.7) (layer "B.Cu") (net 12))
 (segment (start 115.6 35) (end 115.6 32.1) (width 0.7) (layer "B.Cu") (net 1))
 (segment (start 115.6 32.1) (end 115.5 32) (width 0.7) (layer "B.Cu") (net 1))
 (segment (start 110.52 35) (end 110.52 32.1) (width 0.7) (layer "B.Cu") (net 3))
 (segment (start 110.52 32.1) (end 110.42 32) (width 0.7) (layer "B.Cu") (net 3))
 (segment (start 107.98 35) (end 107.98 32.1) (width 0.7) (layer "B.Cu") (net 4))
 (segment (start 107.98 32.1) (end 107.88 32) (width 0.7) (layer "B.Cu") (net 4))
 (segment (start 113.06 32.1) (end 112.96 32) (width 0.7) (layer "B.Cu") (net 2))
 (segment (start 113.06 35) (end 113.06 32.1) (width 0.7) (layer "B.Cu") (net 2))
 (segment (start 103.9 67) (end 104.115 67) (width 0.7) (layer "B.Cu") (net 11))
 (segment (start 95 66.8) (end 103.7 66.8) (width 0.7) (layer "B.Cu") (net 11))
 (segment (start 104.115 67) (end 104.135 66.98) (width 0.7) (layer "B.Cu") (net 11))
 (segment (start 103.865 77.35) (end 103.865 67.035) (width 0.7) (layer "B.Cu") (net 11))
 (segment (start 104.135 66.98) (end 105.9 66.98) (width 0.7) (layer "B.Cu") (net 11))
 (segment (start 103.865 67.035) (end 103.9 67) (width 0.7) (layer "B.Cu") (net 11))
 (segment (start 103.7 66.8) (end 103.9 67) (width 0.7) (layer "B.Cu") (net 11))
 (segment (start 103.565 77.65) (end 103.865 77.35) (width 0.7) (layer "B.Cu") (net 11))
 (segment (start 107.98 54.1) (end 108.18 54.3) (width 0.7) (layer "B.Cu") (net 8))
 (segment (start 108.18 56.36) (end 108.18 54.3) (width 0.7) (layer "B.Cu") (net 8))
 (segment (start 95 54.1) (end 107.98 54.1) (width 0.7) (layer "B.Cu") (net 8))
 (segment (start 96.01 63.25) (end 95 64.26) (width 0.7) (layer "B.Cu") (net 13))
 (segment (start 109.45 63.25) (end 96.01 63.25) (width 0.7) (layer "B.Cu") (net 13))
 (segment (start 112 65.8) (end 109.45 63.25) (width 0.7) (layer "B.Cu") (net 13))
 (segment (start 110.72 56.36) (end 110.72 39.87) (width 0.7) (layer "B.Cu") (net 9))
 (segment (start 110.72 39.87) (end 109.95 39.1) (width 0.7) (layer "B.Cu") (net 9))
 (segment (start 109.71 38.86) (end 109.95 39.1) (width 0.7) (layer "B.Cu") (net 9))
 (segment (start 95 38.86) (end 109.71 38.86) (width 0.7) (layer "B.Cu") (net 9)))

